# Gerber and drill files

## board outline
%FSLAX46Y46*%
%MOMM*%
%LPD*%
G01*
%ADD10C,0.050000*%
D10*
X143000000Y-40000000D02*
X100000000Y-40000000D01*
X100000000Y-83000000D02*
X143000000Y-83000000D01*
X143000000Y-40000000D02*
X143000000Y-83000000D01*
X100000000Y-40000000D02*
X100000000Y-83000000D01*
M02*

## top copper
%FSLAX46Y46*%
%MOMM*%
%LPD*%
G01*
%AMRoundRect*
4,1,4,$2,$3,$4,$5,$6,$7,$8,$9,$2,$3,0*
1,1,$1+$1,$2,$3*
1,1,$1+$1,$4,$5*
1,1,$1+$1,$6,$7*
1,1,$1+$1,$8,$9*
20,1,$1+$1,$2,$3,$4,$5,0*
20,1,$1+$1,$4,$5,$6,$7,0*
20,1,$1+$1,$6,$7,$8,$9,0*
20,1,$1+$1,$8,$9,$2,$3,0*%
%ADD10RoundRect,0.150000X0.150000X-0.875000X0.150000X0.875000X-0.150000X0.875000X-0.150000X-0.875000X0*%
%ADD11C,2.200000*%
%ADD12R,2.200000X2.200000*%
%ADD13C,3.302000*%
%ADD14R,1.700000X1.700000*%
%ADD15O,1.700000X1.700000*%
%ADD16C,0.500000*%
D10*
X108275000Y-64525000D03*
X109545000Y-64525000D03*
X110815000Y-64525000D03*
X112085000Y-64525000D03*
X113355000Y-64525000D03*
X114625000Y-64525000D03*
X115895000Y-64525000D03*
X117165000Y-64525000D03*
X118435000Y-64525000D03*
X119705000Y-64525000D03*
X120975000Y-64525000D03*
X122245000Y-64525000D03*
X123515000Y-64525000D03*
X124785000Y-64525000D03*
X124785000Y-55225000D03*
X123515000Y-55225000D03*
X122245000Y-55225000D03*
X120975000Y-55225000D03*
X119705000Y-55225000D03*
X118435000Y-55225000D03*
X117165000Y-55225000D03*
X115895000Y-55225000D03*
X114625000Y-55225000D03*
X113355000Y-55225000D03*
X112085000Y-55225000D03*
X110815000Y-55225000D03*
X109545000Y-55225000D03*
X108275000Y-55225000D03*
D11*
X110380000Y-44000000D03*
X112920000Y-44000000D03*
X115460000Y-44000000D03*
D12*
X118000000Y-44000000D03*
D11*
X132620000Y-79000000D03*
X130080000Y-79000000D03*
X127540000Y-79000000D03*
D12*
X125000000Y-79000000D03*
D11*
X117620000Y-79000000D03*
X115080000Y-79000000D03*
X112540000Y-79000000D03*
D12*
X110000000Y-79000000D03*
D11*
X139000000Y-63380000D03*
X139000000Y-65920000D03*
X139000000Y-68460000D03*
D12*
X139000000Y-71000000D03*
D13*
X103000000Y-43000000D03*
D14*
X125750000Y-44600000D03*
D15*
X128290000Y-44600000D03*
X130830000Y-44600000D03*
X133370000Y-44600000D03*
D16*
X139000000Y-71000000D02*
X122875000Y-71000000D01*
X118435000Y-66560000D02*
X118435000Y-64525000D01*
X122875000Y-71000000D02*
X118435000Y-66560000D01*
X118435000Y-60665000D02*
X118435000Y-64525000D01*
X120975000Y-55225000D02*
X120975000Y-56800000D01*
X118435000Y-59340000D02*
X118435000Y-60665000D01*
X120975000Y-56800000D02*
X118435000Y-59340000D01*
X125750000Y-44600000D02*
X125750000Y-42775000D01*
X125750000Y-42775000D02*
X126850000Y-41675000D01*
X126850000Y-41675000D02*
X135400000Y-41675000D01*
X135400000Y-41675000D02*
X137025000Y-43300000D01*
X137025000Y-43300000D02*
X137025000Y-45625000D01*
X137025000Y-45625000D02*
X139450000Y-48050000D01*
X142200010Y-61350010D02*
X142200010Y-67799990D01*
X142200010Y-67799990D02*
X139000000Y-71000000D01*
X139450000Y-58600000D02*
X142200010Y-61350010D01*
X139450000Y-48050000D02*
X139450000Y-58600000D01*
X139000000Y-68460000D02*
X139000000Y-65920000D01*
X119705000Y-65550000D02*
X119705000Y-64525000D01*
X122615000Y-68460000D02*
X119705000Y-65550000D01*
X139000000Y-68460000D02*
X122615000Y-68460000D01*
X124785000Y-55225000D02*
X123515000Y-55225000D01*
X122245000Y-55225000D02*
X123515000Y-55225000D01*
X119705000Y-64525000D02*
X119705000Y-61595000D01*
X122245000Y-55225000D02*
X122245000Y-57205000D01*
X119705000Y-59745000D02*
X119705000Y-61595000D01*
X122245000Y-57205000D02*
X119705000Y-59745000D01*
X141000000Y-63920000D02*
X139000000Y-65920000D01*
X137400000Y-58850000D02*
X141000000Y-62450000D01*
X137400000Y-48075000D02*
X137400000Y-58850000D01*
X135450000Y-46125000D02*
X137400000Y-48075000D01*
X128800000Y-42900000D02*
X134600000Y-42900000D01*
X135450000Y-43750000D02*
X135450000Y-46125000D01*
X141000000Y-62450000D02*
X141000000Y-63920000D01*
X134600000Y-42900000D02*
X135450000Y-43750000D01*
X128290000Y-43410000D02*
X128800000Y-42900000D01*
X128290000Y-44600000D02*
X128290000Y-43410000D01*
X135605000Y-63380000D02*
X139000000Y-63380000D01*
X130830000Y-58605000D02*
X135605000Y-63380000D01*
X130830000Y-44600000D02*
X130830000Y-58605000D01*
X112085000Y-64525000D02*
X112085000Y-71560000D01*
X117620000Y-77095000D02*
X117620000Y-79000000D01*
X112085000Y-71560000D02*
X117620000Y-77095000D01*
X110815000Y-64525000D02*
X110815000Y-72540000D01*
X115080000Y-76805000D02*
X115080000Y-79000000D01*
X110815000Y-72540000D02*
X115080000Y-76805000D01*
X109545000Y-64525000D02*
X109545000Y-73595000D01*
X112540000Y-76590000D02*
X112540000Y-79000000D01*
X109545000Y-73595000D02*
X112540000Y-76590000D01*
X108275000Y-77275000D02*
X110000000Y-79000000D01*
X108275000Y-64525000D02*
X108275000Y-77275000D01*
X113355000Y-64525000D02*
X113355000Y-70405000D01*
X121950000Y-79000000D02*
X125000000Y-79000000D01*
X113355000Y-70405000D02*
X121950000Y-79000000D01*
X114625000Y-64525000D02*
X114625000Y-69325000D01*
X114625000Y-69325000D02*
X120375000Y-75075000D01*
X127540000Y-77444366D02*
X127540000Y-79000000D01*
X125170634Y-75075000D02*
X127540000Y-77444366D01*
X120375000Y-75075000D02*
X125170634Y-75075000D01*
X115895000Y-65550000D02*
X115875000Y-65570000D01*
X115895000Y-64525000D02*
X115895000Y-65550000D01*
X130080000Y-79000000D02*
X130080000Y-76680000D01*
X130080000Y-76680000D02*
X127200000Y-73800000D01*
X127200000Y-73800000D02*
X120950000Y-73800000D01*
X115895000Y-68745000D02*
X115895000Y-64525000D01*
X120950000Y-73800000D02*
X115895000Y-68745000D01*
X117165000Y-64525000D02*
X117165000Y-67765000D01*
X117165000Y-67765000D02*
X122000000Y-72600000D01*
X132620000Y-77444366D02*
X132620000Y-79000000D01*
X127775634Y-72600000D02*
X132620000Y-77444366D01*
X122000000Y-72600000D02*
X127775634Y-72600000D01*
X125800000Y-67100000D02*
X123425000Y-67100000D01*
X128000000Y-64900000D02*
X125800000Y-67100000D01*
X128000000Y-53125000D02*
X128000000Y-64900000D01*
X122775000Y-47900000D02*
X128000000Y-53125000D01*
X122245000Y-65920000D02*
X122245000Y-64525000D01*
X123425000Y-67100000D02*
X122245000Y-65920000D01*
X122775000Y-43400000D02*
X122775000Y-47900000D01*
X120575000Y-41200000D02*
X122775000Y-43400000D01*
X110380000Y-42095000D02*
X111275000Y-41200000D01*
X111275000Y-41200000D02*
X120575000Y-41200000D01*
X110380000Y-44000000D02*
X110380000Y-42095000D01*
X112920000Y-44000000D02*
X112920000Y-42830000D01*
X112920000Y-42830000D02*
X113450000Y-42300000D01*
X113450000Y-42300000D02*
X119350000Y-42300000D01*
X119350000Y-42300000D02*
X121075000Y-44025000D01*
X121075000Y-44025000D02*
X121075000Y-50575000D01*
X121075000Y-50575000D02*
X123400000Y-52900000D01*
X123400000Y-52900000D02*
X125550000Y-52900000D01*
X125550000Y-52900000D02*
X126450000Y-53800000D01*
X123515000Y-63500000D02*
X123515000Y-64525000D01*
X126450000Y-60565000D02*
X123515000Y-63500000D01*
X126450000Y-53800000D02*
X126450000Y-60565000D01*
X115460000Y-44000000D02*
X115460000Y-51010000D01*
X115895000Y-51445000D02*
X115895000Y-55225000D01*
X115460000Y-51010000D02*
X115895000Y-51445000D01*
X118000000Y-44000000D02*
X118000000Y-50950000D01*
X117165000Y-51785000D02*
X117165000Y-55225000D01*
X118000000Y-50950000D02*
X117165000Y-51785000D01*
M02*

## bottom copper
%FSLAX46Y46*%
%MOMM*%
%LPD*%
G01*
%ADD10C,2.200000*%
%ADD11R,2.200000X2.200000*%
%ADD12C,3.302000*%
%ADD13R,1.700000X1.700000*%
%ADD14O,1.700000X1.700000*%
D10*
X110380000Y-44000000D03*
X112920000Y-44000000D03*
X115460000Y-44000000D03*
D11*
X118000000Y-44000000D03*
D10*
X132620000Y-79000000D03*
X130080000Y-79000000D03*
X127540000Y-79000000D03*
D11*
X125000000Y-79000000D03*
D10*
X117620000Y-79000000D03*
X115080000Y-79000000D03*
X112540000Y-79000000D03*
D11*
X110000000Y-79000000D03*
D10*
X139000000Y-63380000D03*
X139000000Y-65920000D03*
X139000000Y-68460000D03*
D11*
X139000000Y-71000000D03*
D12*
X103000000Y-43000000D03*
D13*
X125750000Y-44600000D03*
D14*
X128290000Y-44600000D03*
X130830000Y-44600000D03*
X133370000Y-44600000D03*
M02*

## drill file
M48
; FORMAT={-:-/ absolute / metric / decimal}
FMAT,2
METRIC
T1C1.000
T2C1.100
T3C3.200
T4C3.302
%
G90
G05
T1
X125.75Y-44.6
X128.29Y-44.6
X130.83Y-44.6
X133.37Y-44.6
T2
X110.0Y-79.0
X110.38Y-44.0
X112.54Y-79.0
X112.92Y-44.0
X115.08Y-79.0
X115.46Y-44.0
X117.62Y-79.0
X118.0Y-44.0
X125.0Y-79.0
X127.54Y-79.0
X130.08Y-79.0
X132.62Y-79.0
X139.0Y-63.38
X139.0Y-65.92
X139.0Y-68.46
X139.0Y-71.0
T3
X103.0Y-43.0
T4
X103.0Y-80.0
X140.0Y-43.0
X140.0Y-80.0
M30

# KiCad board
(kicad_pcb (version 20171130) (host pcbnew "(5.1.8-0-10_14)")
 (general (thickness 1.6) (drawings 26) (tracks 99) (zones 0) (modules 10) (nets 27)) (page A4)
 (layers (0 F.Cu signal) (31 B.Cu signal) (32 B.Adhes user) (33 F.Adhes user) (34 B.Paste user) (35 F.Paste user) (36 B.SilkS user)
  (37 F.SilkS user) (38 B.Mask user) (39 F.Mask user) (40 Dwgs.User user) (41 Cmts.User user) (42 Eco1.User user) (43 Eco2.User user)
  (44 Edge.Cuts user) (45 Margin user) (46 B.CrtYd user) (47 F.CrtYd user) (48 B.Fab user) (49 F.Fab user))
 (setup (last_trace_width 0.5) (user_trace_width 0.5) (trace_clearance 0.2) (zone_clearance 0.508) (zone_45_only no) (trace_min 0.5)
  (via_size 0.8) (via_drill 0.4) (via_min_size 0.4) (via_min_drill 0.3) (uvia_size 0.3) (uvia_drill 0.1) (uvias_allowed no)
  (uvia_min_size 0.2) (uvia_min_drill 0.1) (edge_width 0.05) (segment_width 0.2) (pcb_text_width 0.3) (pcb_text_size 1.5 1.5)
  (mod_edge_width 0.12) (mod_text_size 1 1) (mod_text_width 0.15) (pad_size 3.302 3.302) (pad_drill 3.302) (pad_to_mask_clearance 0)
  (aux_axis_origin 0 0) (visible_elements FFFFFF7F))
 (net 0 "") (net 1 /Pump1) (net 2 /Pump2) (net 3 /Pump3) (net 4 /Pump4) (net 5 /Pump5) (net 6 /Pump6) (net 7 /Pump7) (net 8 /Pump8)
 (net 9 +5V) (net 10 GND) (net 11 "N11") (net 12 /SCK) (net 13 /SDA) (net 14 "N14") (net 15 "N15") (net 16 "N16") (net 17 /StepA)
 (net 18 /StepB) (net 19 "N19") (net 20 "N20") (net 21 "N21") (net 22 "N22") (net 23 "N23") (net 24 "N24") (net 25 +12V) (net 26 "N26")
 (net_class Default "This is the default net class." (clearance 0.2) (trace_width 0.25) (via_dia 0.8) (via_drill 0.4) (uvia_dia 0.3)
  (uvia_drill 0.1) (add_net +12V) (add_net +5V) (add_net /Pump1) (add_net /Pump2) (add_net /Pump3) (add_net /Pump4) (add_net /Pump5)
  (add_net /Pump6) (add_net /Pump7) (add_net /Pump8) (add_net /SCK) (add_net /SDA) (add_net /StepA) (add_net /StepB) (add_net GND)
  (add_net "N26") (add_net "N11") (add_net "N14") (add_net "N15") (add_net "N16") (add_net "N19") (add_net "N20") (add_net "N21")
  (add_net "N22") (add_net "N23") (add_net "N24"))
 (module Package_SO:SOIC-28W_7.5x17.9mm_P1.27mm (layer F.Cu) (at 116.53 59.875 90)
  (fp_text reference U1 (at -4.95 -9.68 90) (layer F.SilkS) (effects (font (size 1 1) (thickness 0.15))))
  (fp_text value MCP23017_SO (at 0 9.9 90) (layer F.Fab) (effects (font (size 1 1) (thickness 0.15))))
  (pad 1 smd roundrect (at -4.65 -8.255 90) (size 2.05 0.6) (layers F.Cu F.Paste F.Mask) (roundrect_rratio 0.25) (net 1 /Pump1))
  (pad 2 smd roundrect (at -4.65 -6.985 90) (size 2.05 0.6) (layers F.Cu F.Paste F.Mask) (roundrect_rratio 0.25) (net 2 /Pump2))
  (pad 3 smd roundrect (at -4.65 -5.715 90) (size 2.05 0.6) (layers F.Cu F.Paste F.Mask) (roundrect_rratio 0.25) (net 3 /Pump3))
  (pad 4 smd roundrect (at -4.65 -4.445 90) (size 2.05 0.6) (layers F.Cu F.Paste F.Mask) (roundrect_rratio 0.25) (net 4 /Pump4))
  (pad 5 smd roundrect (at -4.65 -3.175 90) (size 2.05 0.6) (layers F.Cu F.Paste F.Mask) (roundrect_rratio 0.25) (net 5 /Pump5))
  (pad 6 smd roundrect (at -4.65 -1.905 90) (size 2.05 0.6) (layers F.Cu F.Paste F.Mask) (roundrect_rratio 0.25) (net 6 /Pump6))
  (pad 7 smd roundrect (at -4.65 -0.635 90) (size 2.05 0.6) (layers F.Cu F.Paste F.Mask) (roundrect_rratio 0.25) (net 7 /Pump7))
  (pad 8 smd roundrect (at -4.65 0.635 90) (size 2.05 0.6) (layers F.Cu F.Paste F.Mask) (roundrect_rratio 0.25) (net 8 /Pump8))
  (pad 9 smd roundrect (at -4.65 1.905 90) (size 2.05 0.6) (layers F.Cu F.Paste F.Mask) (roundrect_rratio 0.25) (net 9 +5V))
  (pad 10 smd roundrect (at -4.65 3.175 90) (size 2.05 0.6) (layers F.Cu F.Paste F.Mask) (roundrect_rratio 0.25) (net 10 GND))
  (pad 11 smd roundrect (at -4.65 4.445 90) (size 2.05 0.6) (layers F.Cu F.Paste F.Mask) (roundrect_rratio 0.25) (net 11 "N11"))
  (pad 12 smd roundrect (at -4.65 5.715 90) (size 2.05 0.6) (layers F.Cu F.Paste F.Mask) (roundrect_rratio 0.25) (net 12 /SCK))
  (pad 13 smd roundrect (at -4.65 6.985 90) (size 2.05 0.6) (layers F.Cu F.Paste F.Mask) (roundrect_rratio 0.25) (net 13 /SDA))
  (pad 14 smd roundrect (at -4.65 8.255 90) (size 2.05 0.6) (layers F.Cu F.Paste F.Mask) (roundrect_rratio 0.25) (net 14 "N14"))
  (pad 15 smd roundrect (at 4.65 8.255 90) (size 2.05 0.6) (layers F.Cu F.Paste F.Mask) (roundrect_rratio 0.25) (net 10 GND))
  (pad 16 smd roundrect (at 4.65 6.985 90) (size 2.05 0.6) (layers F.Cu F.Paste F.Mask) (roundrect_rratio 0.25) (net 10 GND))
  (pad 17 smd roundrect (at 4.65 5.715 90) (size 2.05 0.6) (layers F.Cu F.Paste F.Mask) (roundrect_rratio 0.25) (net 10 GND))
  (pad 18 smd roundrect (at 4.65 4.445 90) (size 2.05 0.6) (layers F.Cu F.Paste F.Mask) (roundrect_rratio 0.25) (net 9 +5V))
  (pad 19 smd roundrect (at 4.65 3.175 90) (size 2.05 0.6) (layers F.Cu F.Paste F.Mask) (roundrect_rratio 0.25) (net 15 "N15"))
  (pad 20 smd roundrect (at 4.65 1.905 90) (size 2.05 0.6) (layers F.Cu F.Paste F.Mask) (roundrect_rratio 0.25) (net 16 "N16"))
  (pad 21 smd roundrect (at 4.65 0.635 90) (size 2.05 0.6) (layers F.Cu F.Paste F.Mask) (roundrect_rratio 0.25) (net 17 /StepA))
  (pad 22 smd roundrect (at 4.65 -0.635 90) (size 2.05 0.6) (layers F.Cu F.Paste F.Mask) (roundrect_rratio 0.25) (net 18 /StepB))
  (pad 23 smd roundrect (at 4.65 -1.905 90) (size 2.05 0.6) (layers F.Cu F.Paste F.Mask) (roundrect_rratio 0.25) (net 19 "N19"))
  (pad 24 smd roundrect (at 4.65 -3.175 90) (size 2.05 0.6) (layers F.Cu F.Paste F.Mask) (roundrect_rratio 0.25) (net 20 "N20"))
  (pad 25 smd roundrect (at 4.65 -4.445 90) (size 2.05 0.6) (layers F.Cu F.Paste F.Mask) (roundrect_rratio 0.25) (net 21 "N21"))
  (pad 26 smd roundrect (at 4.65 -5.715 90) (size 2.05 0.6) (layers F.Cu F.Paste F.Mask) (roundrect_rratio 0.25) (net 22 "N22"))
  (pad 27 smd roundrect (at 4.65 -6.985 90) (size 2.05 0.6) (layers F.Cu F.Paste F.Mask) (roundrect_rratio 0.25) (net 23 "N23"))
  (pad 28 smd roundrect (at 4.65 -8.255 90) (size 2.05 0.6) (layers F.Cu F.Paste F.Mask) (roundrect_rratio 0.25) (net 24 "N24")))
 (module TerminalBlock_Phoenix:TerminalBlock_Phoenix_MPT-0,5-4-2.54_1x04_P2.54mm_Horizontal (layer F.Cu) (at 118 44 180)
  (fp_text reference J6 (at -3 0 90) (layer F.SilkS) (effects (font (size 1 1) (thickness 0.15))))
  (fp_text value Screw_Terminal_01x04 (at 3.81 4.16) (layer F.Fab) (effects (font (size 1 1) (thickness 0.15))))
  (pad 4 thru_hole circle (at 7.62 0 180) (size 2.2 2.2) (drill 1.1) (layers *.Cu *.Mask) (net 12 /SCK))
  (pad 3 thru_hole circle (at 5.08 0 180) (size 2.2 2.2) (drill 1.1) (layers *.Cu *.Mask) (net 13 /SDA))
  (pad 2 thru_hole circle (at 2.54 0 180) (size 2.2 2.2) (drill 1.1) (layers *.Cu *.Mask) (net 18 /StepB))
  (pad 1 thru_hole rect (at 0 0 180) (size 2.2 2.2) (drill 1.1) (layers *.Cu *.Mask) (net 17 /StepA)))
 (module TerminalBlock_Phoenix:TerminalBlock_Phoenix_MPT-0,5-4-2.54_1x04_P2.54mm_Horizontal (layer F.Cu) (at 125 79)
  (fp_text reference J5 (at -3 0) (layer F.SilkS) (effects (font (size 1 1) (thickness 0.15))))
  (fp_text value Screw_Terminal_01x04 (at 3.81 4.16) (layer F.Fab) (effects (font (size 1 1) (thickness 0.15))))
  (pad 4 thru_hole circle (at 7.62 0) (size 2.2 2.2) (drill 1.1) (layers *.Cu *.Mask) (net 8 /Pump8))
  (pad 3 thru_hole circle (at 5.08 0) (size 2.2 2.2) (drill 1.1) (layers *.Cu *.Mask) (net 7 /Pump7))
  (pad 2 thru_hole circle (at 2.54 0) (size 2.2 2.2) (drill 1.1) (layers *.Cu *.Mask) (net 6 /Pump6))
  (pad 1 thru_hole rect (at 0 0) (size 2.2 2.2) (drill 1.1) (layers *.Cu *.Mask) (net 5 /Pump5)))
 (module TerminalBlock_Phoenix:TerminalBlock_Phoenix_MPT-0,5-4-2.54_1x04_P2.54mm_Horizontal (layer F.Cu) (at 110 79)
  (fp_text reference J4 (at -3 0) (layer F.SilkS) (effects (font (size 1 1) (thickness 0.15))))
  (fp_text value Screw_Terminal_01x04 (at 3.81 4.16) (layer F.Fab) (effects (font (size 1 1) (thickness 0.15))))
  (pad 4 thru_hole circle (at 7.62 0) (size 2.2 2.2) (drill 1.1) (layers *.Cu *.Mask) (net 4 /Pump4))
  (pad 3 thru_hole circle (at 5.08 0) (size 2.2 2.2) (drill 1.1) (layers *.Cu *.Mask) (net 3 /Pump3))
  (pad 2 thru_hole circle (at 2.54 0) (size 2.2 2.2) (drill 1.1) (layers *.Cu *.Mask) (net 2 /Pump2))
  (pad 1 thru_hole rect (at 0 0) (size 2.2 2.2) (drill 1.1) (layers *.Cu *.Mask) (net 1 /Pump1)))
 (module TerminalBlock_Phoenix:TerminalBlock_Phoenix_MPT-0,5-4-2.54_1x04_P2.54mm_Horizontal (layer F.Cu) (at 139 71 90)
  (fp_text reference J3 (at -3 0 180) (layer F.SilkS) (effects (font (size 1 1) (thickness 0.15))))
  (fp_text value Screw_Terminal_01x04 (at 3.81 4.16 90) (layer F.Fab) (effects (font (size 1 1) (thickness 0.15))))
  (pad 4 thru_hole circle (at 7.62 0 90) (size 2.2 2.2) (drill 1.1) (layers *.Cu *.Mask) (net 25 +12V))
  (pad 3 thru_hole circle (at 5.08 0 90) (size 2.2 2.2) (drill 1.1) (layers *.Cu *.Mask) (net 10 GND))
  (pad 2 thru_hole circle (at 2.54 0 90) (size 2.2 2.2) (drill 1.1) (layers *.Cu *.Mask) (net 10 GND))
  (pad 1 thru_hole rect (at 0 0 90) (size 2.2 2.2) (drill 1.1) (layers *.Cu *.Mask) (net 9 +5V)))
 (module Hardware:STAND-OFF (layer F.Cu) (at 140 80)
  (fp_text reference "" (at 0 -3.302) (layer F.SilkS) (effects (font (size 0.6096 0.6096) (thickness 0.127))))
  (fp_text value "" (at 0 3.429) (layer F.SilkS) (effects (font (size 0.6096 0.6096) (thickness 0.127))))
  (pad "" np_thru_hole circle (at 0 0) (size 3.302 3.302) (drill 3.302) (layers *.Cu *.Mask) (solder_mask_margin 0.1016)))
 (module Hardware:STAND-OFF (layer F.Cu) (at 103 80)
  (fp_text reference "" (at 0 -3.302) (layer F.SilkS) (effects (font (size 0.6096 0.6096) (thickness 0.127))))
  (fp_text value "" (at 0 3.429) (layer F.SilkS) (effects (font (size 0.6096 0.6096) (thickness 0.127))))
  (pad "" np_thru_hole circle (at 0 0) (size 3.302 3.302) (drill 3.302) (layers *.Cu *.Mask) (solder_mask_margin 0.1016)))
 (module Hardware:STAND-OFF (layer F.Cu) (at 140 43)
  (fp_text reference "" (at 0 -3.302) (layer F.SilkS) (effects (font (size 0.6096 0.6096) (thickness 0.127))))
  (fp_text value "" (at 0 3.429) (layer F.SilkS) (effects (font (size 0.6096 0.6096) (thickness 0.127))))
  (pad "" np_thru_hole circle (at 0 0) (size 3.302 3.302) (drill 3.302) (layers *.Cu *.Mask) (solder_mask_margin 0.1016)))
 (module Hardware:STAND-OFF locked (layer F.Cu) (at 103 43)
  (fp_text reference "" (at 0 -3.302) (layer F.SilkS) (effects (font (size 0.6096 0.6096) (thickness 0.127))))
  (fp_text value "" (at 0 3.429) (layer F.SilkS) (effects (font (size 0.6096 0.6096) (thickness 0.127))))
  (pad "" np_thru_hole circle (at 0 0) (size 3.302 3.302) (drill 3.2) (layers *.Cu *.Mask) (solder_mask_margin 0.1016)))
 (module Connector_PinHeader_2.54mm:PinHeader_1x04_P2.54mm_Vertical (layer F.Cu) (at 125.75 44.6 90)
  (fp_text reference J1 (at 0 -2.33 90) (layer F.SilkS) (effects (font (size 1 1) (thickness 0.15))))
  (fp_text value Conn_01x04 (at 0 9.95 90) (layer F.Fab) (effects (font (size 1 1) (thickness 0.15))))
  (pad 1 thru_hole rect (at 0 0 90) (size 1.7 1.7) (drill 1) (layers *.Cu *.Mask) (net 9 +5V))
  (pad 2 thru_hole oval (at 0 2.54 90) (size 1.7 1.7) (drill 1) (layers *.Cu *.Mask) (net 10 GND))
  (pad 3 thru_hole oval (at 0 5.08 90) (size 1.7 1.7) (drill 1) (layers *.Cu *.Mask) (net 25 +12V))
  (pad 4 thru_hole oval (at 0 7.62 90) (size 1.7 1.7) (drill 1) (layers *.Cu *.Mask) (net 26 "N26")))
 (gr_line (start 143 40) (end 100 40) (layer Edge.Cuts) (width 0.05))
 (gr_line (start 100 83) (end 143 83) (layer Edge.Cuts) (width 0.05))
 (gr_line (start 143 40) (end 143 83) (layer Edge.Cuts) (width 0.05))
 (gr_line (start 100 40) (end 100 83) (layer Edge.Cuts) (width 0.05))
 (segment (start 139 71) (end 122.875 71) (width 0.5) (layer F.Cu) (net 9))
 (segment (start 118.435 66.56) (end 118.435 64.525) (width 0.5) (layer F.Cu) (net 9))
 (segment (start 122.875 71) (end 118.435 66.56) (width 0.5) (layer F.Cu) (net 9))
 (segment (start 118.435 60.665) (end 118.435 64.525) (width 0.5) (layer F.Cu) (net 9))
 (segment (start 120.975 55.225) (end 120.975 56.8) (width 0.5) (layer F.Cu) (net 9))
 (segment (start 118.435 59.34) (end 118.435 60.665) (width 0.5) (layer F.Cu) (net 9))
 (segment (start 120.975 56.8) (end 118.435 59.34) (width 0.5) (layer F.Cu) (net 9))
 (segment (start 125.75 44.6) (end 125.75 42.775) (width 0.5) (layer F.Cu) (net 9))
 (segment (start 125.75 42.775) (end 126.85 41.675) (width 0.5) (layer F.Cu) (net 9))
 (segment (start 126.85 41.675) (end 135.4 41.675) (width 0.5) (layer F.Cu) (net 9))
 (segment (start 135.4 41.675) (end 137.025 43.3) (width 0.5) (layer F.Cu) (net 9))
 (segment (start 137.025 43.3) (end 137.025 45.625) (width 0.5) (layer F.Cu) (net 9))
 (segment (start 137.025 45.625) (end 139.45 48.05) (width 0.5) (layer F.Cu) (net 9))
 (segment (start 142.20001 61.35001) (end 142.20001 67.79999) (width 0.5) (layer F.Cu) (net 9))
 (segment (start 142.20001 67.79999) (end 139 71) (width 0.5) (layer F.Cu) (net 9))
 (segment (start 139.45 58.6) (end 142.20001 61.35001) (width 0.5) (layer F.Cu) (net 9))
 (segment (start 139.45 48.05) (end 139.45 58.6) (width 0.5) (layer F.Cu) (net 9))
 (segment (start 139 68.46) (end 139 65.92) (width 0.5) (layer F.Cu) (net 10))
 (segment (start 119.705 65.55) (end 119.705 64.525) (width 0.5) (layer F.Cu) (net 10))
 (segment (start 122.615 68.46) (end 119.705 65.55) (width 0.5) (layer F.Cu) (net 10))
 (segment (start 139 68.46) (end 122.615 68.46) (width 0.5) (layer F.Cu) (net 10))
 (segment (start 124.785 55.225) (end 123.515 55.225) (width 0.5) (layer F.Cu) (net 10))
 (segment (start 122.245 55.225) (end 123.515 55.225) (width 0.5) (layer F.Cu) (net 10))
 (segment (start 119.705 64.525) (end 119.705 61.595) (width 0.5) (layer F.Cu) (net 10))
 (segment (start 122.245 55.225) (end 122.245 57.205) (width 0.5) (layer F.Cu) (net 10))
 (segment (start 119.705 59.745) (end 119.705 61.595) (width 0.5) (layer F.Cu) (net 10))
 (segment (start 122.245 57.205) (end 119.705 59.745) (width 0.5) (layer F.Cu) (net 10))
 (segment (start 141 63.92) (end 139 65.92) (width 0.5) (layer F.Cu) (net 10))
 (segment (start 137.4 58.85) (end 141 62.45) (width 0.5) (layer F.Cu) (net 10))
 (segment (start 137.4 48.075) (end 137.4 58.85) (width 0.5) (layer F.Cu) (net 10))
 (segment (start 135.45 46.125) (end 137.4 48.075) (width 0.5) (layer F.Cu) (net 10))
 (segment (start 128.8 42.9) (end 134.6 42.9) (width 0.5) (layer F.Cu) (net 10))
 (segment (start 135.45 43.75) (end 135.45 46.125) (width 0.5) (layer F.Cu) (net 10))
 (segment (start 141 62.45) (end 141 63.92) (width 0.5) (layer F.Cu) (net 10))
 (segment (start 134.6 42.9) (end 135.45 43.75) (width 0.5) (layer F.Cu) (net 10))
 (segment (start 128.29 43.41) (end 128.8 42.9) (width 0.5) (layer F.Cu) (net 10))
 (segment (start 128.29 44.6) (end 128.29 43.41) (width 0.5) (layer F.Cu) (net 10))
 (segment (start 135.605 63.38) (end 139 63.38) (width 0.5) (layer F.Cu) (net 25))
 (segment (start 130.83 58.605) (end 135.605 63.38) (width 0.5) (layer F.Cu) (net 25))
 (segment (start 130.83 44.6) (end 130.83 58.605) (width 0.5) (layer F.Cu) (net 25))
 (segment (start 112.085 64.525) (end 112.085 71.56) (width 0.5) (layer F.Cu) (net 4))
 (segment (start 117.62 77.095) (end 117.62 79) (width 0.5) (layer F.Cu) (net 4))
 (segment (start 112.085 71.56) (end 117.62 77.095) (width 0.5) (layer F.Cu) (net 4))
 (segment (start 110.815 64.525) (end 110.815 72.54) (width 0.5) (layer F.Cu) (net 3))
 (segment (start 115.08 76.805) (end 115.08 79) (width 0.5) (layer F.Cu) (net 3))
 (segment (start 110.815 72.54) (end 115.08 76.805) (width 0.5) (layer F.Cu) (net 3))
 (segment (start 109.545 64.525) (end 109.545 73.595) (width 0.5) (layer F.Cu) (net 2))
 (segment (start 112.54 76.59) (end 112.54 79) (width 0.5) (layer F.Cu) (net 2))
 (segment (start 109.545 73.595) (end 112.54 76.59) (width 0.5) (layer F.Cu) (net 2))
 (segment (start 108.275 77.275) (end 110 79) (width 0.5) (layer F.Cu) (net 1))
 (segment (start 108.275 64.525) (end 108.275 77.275) (width 0.5) (layer F.Cu) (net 1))
 (segment (start 113.355 64.525) (end 113.355 70.405) (width 0.5) (layer F.Cu) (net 5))
 (segment (start 121.95 79) (end 125 79) (width 0.5) (layer F.Cu) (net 5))
 (segment (start 113.355 70.405) (end 121.95 79) (width 0.5) (layer F.Cu) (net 5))
 (segment (start 114.625 64.525) (end 114.625 69.325) (width 0.5) (layer F.Cu) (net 6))
 (segment (start 114.625 69.325) (end 120.375 75.075) (width 0.5) (layer F.Cu) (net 6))
 (segment (start 127.54 77.444366) (end 127.54 79) (width 0.5) (layer F.Cu) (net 6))
 (segment (start 125.170634 75.075) (end 127.54 77.444366) (width 0.5) (layer F.Cu) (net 6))
 (segment (start 120.375 75.075) (end 125.170634 75.075) (width 0.5) (layer F.Cu) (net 6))
 (segment (start 115.895 65.55) (end 115.875 65.57) (width 0.5) (layer F.Cu) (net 7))
 (segment (start 115.895 64.525) (end 115.895 65.55) (width 0.5) (layer F.Cu) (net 7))
 (segment (start 130.08 79) (end 130.08 76.68) (width 0.5) (layer F.Cu) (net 7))
 (segment (start 130.08 76.68) (end 127.2 73.8) (width 0.5) (layer F.Cu) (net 7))
 (segment (start 127.2 73.8) (end 120.95 73.8) (width 0.5) (layer F.Cu) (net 7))
 (segment (start 115.895 68.745) (end 115.895 64.525) (width 0.5) (layer F.Cu) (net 7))
 (segment (start 120.95 73.8) (end 115.895 68.745) (width 0.5) (layer F.Cu) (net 7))
 (segment (start 117.165 64.525) (end 117.165 67.765) (width 0.5) (layer F.Cu) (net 8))
 (segment (start 117.165 67.765) (end 122 72.6) (width 0.5) (layer F.Cu) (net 8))
 (segment (start 132.62 77.444366) (end 132.62 79) (width 0.5) (layer F.Cu) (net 8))
 (segment (start 127.775634 72.6) (end 132.62 77.444366) (width 0.5) (layer F.Cu) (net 8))
 (segment (start 122 72.6) (end 127.775634 72.6) (width 0.5) (layer F.Cu) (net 8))
 (segment (start 125.8 67.1) (end 123.425 67.1) (width 0.5) (layer F.Cu) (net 12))
 (segment (start 128 64.9) (end 125.8 67.1) (width 0.5) (layer F.Cu) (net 12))
 (segment (start 128 53.125) (end 128 64.9) (width 0.5) (layer F.Cu) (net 12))
 (segment (start 122.775 47.9) (end 128 53.125) (width 0.5) (layer F.Cu) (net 12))
 (segment (start 122.245 65.92) (end 122.245 64.525) (width 0.5) (layer F.Cu) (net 12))
 (segment (start 123.425 67.1) (end 122.245 65.92) (width 0.5) (layer F.Cu) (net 12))
 (segment (start 122.775 43.4) (end 122.775 47.9) (width 0.5) (layer F.Cu) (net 12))
 (segment (start 120.575 41.2) (end 122.775 43.4) (width 0.5) (layer F.Cu) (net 12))
 (segment (start 110.38 42.095) (end 111.275 41.2) (width 0.5) (layer F.Cu) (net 12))
 (segment (start 111.275 41.2) (end 120.575 41.2) (width 0.5) (layer F.Cu) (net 12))
 (segment (start 110.38 44) (end 110.38 42.095) (width 0.5) (layer F.Cu) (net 12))
 (segment (start 112.92 44) (end 112.92 42.83) (width 0.5) (layer F.Cu) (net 13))
 (segment (start 112.92 42.83) (end 113.45 42.3) (width 0.5) (layer F.Cu) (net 13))
 (segment (start 113.45 42.3) (end 119.35 42.3) (width 0.5) (layer F.Cu) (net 13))
 (segment (start 119.35 42.3) (end 121.075 44.025) (width 0.5) (layer F.Cu) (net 13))
 (segment (start 121.075 44.025) (end 121.075 50.575) (width 0.5) (layer F.Cu) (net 13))
 (segment (start 121.075 50.575) (end 123.4 52.9) (width 0.5) (layer F.Cu) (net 13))
 (segment (start 123.4 52.9) (end 125.55 52.9) (width 0.5) (layer F.Cu) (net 13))
 (segment (start 125.55 52.9) (end 126.45 53.8) (width 0.5) (layer F.Cu) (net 13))
 (segment (start 123.515 63.5) (end 123.515 64.525) (width 0.5) (layer F.Cu) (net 13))
 (segment (start 126.45 60.565) (end 123.515 63.5) (width 0.5) (layer F.Cu) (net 13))
 (segment (start 126.45 53.8) (end 126.45 60.565) (width 0.5) (layer F.Cu) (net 13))
 (segment (start 115.46 44) (end 115.46 51.01) (width 0.5) (layer F.Cu) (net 18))
 (segment (start 115.895 51.445) (end 115.895 55.225) (width 0.5) (layer F.Cu) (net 18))
 (segment (start 115.46 51.01) (end 115.895 51.445) (width 0.5) (layer F.Cu) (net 18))
 (segment (start 118 44) (end 118 50.95) (width 0.5) (layer F.Cu) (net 17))
 (segment (start 117.165 51.785) (end 117.165 55.225) (width 0.5) (layer F.Cu) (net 17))
 (segment (start 118 50.95) (end 117.165 51.785) (width 0.5) (layer F.Cu) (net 17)))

